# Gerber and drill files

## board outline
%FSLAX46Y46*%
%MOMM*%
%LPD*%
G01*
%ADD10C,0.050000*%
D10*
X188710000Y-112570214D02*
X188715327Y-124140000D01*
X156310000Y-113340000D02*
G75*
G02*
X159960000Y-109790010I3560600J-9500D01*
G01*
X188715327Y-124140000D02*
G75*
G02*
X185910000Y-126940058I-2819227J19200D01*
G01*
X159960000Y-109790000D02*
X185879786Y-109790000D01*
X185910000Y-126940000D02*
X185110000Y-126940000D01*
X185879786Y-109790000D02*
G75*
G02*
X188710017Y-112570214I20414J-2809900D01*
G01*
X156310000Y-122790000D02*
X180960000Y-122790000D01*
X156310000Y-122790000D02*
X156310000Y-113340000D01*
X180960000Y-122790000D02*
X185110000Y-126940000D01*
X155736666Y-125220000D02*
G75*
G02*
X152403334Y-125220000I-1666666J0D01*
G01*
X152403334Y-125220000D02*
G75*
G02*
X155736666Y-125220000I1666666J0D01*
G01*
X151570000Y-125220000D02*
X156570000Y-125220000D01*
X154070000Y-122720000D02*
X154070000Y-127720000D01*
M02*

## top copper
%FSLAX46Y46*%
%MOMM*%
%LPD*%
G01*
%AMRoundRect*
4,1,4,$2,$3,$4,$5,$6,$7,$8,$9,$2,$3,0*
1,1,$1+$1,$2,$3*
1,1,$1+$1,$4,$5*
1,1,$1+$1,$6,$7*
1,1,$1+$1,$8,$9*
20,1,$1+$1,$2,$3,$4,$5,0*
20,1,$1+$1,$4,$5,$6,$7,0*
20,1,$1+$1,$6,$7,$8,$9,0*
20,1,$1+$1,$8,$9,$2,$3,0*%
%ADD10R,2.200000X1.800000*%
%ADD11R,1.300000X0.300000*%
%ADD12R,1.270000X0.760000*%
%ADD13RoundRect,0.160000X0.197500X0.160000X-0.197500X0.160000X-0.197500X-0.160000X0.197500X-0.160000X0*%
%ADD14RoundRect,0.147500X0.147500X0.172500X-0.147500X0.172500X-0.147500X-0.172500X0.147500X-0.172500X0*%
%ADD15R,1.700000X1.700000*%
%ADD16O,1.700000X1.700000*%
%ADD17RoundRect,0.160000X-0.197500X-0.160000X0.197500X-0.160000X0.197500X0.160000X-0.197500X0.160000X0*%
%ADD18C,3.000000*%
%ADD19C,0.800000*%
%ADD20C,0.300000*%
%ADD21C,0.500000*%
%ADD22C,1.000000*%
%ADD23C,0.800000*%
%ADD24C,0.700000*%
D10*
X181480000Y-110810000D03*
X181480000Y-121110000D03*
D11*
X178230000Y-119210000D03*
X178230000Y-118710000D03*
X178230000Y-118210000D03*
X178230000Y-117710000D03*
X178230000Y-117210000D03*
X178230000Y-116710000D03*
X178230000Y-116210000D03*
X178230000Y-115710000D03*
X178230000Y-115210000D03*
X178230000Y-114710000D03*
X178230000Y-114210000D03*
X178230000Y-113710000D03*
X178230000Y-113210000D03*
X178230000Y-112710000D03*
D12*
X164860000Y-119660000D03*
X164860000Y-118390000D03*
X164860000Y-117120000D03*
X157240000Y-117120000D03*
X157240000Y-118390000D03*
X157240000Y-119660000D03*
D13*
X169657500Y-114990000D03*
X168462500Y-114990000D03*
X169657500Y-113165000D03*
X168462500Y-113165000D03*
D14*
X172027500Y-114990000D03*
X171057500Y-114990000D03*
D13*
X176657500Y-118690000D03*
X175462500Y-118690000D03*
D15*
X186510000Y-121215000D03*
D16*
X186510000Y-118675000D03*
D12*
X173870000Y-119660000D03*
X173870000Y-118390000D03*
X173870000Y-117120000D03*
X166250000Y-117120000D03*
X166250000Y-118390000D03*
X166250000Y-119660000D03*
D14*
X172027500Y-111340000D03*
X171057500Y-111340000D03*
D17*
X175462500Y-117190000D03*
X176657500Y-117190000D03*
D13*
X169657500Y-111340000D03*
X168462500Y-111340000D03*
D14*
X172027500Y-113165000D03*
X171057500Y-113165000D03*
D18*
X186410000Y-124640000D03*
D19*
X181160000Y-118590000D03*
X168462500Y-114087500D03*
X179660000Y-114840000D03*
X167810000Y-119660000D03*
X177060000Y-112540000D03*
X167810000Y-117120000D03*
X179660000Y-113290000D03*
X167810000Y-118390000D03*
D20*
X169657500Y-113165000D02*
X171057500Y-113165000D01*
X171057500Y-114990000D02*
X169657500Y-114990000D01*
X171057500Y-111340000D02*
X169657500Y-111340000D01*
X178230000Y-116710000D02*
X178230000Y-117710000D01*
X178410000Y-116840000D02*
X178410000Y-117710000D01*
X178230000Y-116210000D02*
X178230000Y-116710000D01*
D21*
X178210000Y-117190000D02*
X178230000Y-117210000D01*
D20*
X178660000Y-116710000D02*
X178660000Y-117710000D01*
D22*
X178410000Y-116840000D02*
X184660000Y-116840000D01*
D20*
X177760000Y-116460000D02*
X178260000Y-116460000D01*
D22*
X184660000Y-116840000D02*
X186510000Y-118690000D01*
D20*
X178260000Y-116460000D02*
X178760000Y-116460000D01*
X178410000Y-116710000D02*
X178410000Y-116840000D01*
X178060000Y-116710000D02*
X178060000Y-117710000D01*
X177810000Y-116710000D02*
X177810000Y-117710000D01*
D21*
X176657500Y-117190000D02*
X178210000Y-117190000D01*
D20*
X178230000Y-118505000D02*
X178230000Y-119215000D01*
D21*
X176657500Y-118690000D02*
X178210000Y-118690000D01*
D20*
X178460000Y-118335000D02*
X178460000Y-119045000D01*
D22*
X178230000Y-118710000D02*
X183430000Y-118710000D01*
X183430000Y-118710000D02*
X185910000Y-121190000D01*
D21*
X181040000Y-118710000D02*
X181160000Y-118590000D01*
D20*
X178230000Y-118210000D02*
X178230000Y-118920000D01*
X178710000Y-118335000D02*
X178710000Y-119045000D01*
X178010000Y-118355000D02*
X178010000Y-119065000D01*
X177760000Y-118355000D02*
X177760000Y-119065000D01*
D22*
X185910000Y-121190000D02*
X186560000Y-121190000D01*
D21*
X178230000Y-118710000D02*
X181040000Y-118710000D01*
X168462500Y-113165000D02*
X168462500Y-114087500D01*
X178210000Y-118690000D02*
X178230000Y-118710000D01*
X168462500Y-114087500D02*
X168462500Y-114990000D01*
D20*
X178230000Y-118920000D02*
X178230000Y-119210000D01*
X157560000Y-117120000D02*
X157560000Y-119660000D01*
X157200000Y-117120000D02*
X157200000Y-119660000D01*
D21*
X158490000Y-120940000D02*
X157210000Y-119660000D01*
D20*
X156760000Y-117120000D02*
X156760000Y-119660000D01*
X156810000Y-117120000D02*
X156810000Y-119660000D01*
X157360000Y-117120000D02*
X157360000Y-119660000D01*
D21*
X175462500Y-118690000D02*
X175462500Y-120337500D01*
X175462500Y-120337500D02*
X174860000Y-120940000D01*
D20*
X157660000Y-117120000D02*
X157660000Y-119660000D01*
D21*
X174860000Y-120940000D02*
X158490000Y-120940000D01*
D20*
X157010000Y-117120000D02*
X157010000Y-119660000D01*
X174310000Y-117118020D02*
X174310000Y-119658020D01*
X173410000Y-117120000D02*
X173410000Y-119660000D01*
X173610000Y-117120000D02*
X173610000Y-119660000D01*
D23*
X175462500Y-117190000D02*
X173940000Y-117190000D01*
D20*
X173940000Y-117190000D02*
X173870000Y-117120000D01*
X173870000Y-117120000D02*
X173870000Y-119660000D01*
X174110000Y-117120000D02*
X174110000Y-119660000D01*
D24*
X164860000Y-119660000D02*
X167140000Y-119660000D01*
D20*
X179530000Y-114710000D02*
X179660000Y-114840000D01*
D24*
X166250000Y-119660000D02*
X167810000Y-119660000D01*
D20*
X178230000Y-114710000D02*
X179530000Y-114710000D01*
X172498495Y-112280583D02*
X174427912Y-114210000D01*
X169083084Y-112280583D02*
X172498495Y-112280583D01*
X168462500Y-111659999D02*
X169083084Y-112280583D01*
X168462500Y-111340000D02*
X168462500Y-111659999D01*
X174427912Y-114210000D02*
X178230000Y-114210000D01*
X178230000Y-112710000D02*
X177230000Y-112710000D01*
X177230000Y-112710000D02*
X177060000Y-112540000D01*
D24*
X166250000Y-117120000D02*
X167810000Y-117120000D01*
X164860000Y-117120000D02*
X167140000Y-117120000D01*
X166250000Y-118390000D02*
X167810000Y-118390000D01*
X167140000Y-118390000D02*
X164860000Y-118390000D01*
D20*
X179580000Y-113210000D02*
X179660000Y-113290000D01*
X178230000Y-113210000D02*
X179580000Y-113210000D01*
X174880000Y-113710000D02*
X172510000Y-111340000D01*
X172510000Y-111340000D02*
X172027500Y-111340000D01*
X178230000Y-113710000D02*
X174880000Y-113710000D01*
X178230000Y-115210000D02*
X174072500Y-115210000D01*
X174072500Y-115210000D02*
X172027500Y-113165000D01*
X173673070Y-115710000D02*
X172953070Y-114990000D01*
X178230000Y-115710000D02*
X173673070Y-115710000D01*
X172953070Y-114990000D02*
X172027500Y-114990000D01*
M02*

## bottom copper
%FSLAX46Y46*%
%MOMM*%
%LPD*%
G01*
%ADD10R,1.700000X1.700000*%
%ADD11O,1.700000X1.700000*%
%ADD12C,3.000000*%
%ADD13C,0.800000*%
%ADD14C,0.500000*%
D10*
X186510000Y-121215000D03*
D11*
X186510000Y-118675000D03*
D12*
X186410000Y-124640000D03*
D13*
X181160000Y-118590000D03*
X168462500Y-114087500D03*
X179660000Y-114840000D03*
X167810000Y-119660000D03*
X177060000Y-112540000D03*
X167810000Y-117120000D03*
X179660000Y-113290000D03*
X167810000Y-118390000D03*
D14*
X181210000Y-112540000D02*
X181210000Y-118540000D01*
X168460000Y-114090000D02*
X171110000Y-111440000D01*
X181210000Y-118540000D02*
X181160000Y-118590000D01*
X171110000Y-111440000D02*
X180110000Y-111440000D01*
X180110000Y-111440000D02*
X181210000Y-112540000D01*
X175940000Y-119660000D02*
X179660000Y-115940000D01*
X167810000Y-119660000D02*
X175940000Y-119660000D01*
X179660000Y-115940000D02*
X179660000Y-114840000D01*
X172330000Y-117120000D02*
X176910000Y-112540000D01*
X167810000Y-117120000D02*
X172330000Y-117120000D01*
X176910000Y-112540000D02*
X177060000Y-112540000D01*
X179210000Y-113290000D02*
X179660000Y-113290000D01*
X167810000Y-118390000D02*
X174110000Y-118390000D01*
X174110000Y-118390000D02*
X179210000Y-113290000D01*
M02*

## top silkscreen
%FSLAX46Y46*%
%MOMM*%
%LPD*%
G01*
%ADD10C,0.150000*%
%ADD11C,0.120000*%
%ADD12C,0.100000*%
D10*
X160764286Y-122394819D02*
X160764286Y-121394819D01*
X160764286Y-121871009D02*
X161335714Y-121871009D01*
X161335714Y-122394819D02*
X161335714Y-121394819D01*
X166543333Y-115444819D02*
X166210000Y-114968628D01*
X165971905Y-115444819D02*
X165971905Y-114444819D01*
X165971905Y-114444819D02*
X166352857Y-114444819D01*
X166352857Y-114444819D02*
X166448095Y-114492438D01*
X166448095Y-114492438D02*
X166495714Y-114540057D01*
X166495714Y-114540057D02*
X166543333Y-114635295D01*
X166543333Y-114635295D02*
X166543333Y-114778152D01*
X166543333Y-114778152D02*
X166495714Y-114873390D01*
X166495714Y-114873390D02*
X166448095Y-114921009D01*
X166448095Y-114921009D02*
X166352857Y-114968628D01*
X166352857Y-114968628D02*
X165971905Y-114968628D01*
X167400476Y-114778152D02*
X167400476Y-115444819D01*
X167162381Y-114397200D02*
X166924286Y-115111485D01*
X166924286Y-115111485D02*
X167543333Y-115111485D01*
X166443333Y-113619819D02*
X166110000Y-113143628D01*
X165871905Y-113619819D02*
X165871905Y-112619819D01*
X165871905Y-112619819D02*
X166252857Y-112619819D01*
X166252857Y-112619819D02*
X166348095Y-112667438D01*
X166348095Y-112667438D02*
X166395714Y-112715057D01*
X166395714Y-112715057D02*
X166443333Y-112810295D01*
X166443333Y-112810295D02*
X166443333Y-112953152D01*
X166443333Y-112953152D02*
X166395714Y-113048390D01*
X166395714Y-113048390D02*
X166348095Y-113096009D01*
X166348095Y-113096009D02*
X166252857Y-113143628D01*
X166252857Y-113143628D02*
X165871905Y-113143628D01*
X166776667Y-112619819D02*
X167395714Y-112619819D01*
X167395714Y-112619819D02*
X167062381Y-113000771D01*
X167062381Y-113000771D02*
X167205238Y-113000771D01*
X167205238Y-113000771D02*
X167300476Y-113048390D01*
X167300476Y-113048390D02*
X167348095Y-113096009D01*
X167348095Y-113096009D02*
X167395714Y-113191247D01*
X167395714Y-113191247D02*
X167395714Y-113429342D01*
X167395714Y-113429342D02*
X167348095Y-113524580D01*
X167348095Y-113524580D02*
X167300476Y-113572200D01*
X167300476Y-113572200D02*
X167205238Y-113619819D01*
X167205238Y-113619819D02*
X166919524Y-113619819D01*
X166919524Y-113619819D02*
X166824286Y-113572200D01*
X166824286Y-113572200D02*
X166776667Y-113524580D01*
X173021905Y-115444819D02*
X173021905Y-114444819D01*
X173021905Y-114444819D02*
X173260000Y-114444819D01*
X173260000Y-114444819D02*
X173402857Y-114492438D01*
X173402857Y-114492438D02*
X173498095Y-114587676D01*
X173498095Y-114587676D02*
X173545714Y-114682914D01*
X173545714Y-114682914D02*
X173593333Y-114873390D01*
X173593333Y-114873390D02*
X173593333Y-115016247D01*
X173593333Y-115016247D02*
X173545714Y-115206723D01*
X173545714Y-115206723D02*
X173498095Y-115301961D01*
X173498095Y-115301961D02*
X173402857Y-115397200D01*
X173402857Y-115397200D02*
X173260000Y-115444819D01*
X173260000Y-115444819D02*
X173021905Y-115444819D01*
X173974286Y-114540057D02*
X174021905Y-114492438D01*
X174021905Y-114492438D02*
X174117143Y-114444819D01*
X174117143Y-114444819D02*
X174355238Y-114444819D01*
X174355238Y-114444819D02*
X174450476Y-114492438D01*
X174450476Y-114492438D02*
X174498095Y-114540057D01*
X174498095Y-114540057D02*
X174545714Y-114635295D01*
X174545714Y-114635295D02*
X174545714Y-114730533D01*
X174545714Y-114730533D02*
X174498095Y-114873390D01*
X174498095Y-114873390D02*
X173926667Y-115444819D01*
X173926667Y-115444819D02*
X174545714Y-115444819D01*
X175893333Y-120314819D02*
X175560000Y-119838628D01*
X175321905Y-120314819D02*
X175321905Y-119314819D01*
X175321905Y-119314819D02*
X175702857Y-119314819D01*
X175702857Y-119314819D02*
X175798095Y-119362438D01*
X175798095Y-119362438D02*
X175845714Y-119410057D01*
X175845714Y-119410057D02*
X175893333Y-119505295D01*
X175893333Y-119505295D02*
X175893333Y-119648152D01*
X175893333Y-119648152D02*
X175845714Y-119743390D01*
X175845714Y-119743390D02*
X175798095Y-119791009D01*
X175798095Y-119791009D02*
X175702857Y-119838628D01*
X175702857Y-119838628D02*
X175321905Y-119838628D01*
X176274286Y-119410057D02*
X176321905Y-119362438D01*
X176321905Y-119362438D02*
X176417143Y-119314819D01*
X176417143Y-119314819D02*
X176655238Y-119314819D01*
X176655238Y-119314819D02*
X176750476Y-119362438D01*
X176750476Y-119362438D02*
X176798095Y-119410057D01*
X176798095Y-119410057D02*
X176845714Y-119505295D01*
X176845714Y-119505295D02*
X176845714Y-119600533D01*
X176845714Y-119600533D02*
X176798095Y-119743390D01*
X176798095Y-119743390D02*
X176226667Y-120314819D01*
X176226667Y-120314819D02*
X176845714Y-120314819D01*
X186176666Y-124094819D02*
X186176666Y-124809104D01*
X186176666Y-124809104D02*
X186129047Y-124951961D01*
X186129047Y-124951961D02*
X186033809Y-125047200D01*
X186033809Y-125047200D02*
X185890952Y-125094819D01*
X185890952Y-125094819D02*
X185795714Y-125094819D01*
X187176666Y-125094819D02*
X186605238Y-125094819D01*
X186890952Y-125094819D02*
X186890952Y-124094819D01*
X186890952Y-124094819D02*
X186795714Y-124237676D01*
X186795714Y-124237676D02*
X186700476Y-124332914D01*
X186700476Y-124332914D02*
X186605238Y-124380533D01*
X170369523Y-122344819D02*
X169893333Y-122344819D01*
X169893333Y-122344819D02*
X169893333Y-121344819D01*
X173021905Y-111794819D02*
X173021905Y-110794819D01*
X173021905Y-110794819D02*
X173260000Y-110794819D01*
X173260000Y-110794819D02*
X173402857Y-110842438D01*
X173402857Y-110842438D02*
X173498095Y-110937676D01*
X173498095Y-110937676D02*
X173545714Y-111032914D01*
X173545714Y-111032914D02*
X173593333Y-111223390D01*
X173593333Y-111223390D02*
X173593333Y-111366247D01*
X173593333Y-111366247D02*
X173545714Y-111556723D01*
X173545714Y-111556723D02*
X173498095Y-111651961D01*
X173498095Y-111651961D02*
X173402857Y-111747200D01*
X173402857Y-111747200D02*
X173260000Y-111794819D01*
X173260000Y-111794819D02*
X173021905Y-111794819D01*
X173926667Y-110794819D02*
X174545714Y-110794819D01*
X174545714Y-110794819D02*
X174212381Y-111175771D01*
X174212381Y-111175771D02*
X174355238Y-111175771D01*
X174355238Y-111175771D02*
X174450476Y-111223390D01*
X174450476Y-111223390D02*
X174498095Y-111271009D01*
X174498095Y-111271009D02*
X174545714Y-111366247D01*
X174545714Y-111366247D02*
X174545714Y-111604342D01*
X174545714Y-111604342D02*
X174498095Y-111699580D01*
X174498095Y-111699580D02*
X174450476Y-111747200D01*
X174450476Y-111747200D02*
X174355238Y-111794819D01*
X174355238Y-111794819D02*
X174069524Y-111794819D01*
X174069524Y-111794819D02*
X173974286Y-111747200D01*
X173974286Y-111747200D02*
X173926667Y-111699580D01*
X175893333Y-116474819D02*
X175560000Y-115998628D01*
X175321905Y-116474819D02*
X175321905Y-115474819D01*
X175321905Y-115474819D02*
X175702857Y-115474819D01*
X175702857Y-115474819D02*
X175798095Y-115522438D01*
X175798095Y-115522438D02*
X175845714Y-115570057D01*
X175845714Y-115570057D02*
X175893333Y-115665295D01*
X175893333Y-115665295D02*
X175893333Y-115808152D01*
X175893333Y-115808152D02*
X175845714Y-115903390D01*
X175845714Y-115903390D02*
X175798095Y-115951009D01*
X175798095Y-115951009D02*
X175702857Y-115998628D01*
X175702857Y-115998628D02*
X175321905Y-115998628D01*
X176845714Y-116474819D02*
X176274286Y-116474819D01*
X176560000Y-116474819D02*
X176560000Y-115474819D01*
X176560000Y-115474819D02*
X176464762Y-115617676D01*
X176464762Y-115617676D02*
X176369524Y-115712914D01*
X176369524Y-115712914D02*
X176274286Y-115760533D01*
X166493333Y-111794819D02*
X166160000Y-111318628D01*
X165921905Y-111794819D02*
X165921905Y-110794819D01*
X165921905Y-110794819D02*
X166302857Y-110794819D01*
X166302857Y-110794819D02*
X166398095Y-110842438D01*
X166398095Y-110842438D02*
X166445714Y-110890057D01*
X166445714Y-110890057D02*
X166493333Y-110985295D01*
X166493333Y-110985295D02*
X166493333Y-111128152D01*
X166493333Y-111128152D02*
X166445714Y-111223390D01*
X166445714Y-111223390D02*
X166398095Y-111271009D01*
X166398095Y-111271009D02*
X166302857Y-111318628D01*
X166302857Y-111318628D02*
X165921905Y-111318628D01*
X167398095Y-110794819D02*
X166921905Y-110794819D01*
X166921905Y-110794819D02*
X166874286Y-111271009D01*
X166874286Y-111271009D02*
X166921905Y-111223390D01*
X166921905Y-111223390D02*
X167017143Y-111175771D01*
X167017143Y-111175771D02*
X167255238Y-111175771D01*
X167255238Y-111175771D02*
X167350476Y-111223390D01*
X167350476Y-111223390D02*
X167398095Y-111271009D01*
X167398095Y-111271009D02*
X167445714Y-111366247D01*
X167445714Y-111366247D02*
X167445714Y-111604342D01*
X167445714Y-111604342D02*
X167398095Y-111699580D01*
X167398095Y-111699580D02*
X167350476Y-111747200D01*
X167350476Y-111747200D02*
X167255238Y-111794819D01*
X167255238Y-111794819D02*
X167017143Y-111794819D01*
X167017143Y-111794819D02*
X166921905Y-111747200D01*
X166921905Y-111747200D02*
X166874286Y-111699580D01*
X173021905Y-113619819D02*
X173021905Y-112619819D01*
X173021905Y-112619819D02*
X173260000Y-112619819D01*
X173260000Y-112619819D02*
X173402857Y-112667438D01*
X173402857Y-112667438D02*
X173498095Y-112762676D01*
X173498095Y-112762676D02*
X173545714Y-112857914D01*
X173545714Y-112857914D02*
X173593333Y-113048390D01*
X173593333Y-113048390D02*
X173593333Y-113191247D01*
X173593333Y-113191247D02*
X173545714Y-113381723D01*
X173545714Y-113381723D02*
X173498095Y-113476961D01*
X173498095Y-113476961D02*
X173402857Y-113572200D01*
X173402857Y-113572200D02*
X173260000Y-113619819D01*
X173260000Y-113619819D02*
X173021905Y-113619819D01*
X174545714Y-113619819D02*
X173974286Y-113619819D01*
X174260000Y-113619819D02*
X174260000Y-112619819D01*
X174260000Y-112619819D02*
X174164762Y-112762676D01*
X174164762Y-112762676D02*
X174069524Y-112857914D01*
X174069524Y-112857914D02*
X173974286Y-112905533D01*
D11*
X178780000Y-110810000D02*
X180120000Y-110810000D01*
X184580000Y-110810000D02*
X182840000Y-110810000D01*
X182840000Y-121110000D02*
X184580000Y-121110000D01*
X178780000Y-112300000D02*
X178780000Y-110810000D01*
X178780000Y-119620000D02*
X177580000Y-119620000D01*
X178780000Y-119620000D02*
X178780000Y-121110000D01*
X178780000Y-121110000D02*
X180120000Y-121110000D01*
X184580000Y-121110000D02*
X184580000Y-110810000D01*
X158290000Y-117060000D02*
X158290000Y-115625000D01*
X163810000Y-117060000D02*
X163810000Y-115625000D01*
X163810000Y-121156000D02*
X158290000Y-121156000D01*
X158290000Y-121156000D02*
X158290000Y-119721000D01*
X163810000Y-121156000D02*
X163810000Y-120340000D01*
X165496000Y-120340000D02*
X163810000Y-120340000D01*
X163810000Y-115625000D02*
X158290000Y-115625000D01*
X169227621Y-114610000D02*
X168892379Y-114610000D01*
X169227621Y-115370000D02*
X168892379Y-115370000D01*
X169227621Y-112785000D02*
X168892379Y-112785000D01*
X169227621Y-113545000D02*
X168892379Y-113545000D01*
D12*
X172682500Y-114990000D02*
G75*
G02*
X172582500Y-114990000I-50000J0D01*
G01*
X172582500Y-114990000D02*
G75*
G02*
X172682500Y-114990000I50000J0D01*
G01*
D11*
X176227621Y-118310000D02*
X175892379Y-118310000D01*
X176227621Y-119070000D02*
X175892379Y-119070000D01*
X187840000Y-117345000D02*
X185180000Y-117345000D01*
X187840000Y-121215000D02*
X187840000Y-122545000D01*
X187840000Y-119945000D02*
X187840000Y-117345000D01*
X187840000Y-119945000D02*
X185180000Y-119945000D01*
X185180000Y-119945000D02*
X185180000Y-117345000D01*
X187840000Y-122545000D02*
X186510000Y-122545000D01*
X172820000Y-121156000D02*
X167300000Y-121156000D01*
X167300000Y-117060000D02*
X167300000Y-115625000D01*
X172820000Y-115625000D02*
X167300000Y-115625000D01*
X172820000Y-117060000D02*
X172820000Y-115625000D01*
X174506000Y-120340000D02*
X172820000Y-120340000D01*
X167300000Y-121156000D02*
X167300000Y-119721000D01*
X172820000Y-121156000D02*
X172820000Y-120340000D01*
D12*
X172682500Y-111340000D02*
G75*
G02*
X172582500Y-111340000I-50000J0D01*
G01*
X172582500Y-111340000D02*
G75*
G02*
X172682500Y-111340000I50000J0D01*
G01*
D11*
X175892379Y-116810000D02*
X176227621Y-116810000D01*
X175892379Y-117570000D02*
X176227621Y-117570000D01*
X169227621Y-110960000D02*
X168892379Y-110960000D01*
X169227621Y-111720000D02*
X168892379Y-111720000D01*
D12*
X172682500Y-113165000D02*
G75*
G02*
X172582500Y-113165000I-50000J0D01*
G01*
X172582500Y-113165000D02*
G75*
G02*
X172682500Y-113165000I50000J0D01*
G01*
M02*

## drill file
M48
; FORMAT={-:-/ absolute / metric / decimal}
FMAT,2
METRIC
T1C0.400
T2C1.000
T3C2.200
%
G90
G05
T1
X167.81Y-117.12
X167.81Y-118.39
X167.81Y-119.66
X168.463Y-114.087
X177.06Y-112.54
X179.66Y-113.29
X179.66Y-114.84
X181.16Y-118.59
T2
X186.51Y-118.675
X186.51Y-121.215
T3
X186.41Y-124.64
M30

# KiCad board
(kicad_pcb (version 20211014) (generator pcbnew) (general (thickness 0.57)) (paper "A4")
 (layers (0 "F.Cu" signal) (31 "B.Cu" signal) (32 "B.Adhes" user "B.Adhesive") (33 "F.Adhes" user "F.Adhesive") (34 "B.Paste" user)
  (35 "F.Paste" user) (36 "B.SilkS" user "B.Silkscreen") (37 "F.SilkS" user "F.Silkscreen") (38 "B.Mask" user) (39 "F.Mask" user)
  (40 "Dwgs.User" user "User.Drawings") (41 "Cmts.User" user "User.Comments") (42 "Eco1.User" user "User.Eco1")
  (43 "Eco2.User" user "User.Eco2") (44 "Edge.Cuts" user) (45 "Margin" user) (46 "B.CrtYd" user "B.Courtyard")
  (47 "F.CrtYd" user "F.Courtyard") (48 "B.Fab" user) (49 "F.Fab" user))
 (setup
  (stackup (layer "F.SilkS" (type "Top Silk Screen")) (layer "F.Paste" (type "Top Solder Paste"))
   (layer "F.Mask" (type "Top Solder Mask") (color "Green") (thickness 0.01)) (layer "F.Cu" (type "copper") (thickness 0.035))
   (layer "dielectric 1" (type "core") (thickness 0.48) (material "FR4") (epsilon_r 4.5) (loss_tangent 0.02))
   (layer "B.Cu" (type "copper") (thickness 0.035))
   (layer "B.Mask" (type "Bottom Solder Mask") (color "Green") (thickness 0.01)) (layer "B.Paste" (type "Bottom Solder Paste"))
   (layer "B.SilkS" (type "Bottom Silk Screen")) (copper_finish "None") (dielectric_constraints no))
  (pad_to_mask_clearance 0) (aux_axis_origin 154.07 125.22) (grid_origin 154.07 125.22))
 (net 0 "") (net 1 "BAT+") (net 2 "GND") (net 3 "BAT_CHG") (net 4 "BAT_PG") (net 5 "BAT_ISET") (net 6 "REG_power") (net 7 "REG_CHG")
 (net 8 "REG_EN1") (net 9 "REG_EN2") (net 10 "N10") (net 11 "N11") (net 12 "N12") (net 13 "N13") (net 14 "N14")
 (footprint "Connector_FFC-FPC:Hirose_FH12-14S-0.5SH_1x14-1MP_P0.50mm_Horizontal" (layer "F.Cu") (at 180.08 115.96 90)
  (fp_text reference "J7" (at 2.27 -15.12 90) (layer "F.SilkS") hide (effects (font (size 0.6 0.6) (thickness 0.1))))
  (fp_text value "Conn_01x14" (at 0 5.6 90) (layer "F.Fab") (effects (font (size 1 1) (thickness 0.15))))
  (fp_line (start 5.15 -1.3) (end 5.15 0.04) (layer "F.SilkS") (width 0.12))
  (fp_line (start 5.15 4.5) (end 5.15 2.76) (layer "F.SilkS") (width 0.12))
  (fp_line (start -5.15 2.76) (end -5.15 4.5) (layer "F.SilkS") (width 0.12))
  (fp_line (start 3.66 -1.3) (end 5.15 -1.3) (layer "F.SilkS") (width 0.12))
  (fp_line (start -3.66 -1.3) (end -3.66 -2.5) (layer "F.SilkS") (width 0.12))
  (fp_line (start -3.66 -1.3) (end -5.15 -1.3) (layer "F.SilkS") (width 0.12))
  (fp_line (start -5.15 -1.3) (end -5.15 0.04) (layer "F.SilkS") (width 0.12))
  (fp_line (start -5.15 4.5) (end 5.15 4.5) (layer "F.SilkS") (width 0.12))
  (pad "" smd rect (at 5.15 1.4 90) (size 1.8 2.2) (layers "F.Cu" "F.Paste" "F.Mask"))
  (pad "" smd rect (at -5.15 1.4 90) (size 1.8 2.2) (layers "F.Cu" "F.Paste" "F.Mask"))
  (pad "1" smd rect (at -3.25 -1.85 90) (size 0.3 1.3) (layers "F.Cu" "F.Paste" "F.Mask") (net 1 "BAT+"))
  (pad "2" smd rect (at -2.75 -1.85 90) (size 0.3 1.3) (layers "F.Cu" "F.Paste" "F.Mask") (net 1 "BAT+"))
  (pad "3" smd rect (at -2.25 -1.85 90) (size 0.3 1.3) (layers "F.Cu" "F.Paste" "F.Mask") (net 1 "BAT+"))
  (pad "4" smd rect (at -1.75 -1.85 90) (size 0.3 1.3) (layers "F.Cu" "F.Paste" "F.Mask") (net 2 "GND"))
  (pad "5" smd rect (at -1.25 -1.85 90) (size 0.3 1.3) (layers "F.Cu" "F.Paste" "F.Mask") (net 2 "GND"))
  (pad "6" smd rect (at -0.75 -1.85 90) (size 0.3 1.3) (layers "F.Cu" "F.Paste" "F.Mask") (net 2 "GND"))
  (pad "7" smd rect (at -0.25 -1.85 90) (size 0.3 1.3) (layers "F.Cu" "F.Paste" "F.Mask") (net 2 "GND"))
  (pad "8" smd rect (at 0.25 -1.85 90) (size 0.3 1.3) (layers "F.Cu" "F.Paste" "F.Mask") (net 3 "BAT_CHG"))
  (pad "9" smd rect (at 0.75 -1.85 90) (size 0.3 1.3) (layers "F.Cu" "F.Paste" "F.Mask") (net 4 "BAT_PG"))
  (pad "10" smd rect (at 1.25 -1.85 90) (size 0.3 1.3) (layers "F.Cu" "F.Paste" "F.Mask") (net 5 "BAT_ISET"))
  (pad "11" smd rect (at 1.75 -1.85 90) (size 0.3 1.3) (layers "F.Cu" "F.Paste" "F.Mask") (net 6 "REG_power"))
  (pad "12" smd rect (at 2.25 -1.85 90) (size 0.3 1.3) (layers "F.Cu" "F.Paste" "F.Mask") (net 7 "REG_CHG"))
  (pad "13" smd rect (at 2.75 -1.85 90) (size 0.3 1.3) (layers "F.Cu" "F.Paste" "F.Mask") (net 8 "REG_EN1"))
  (pad "14" smd rect (at 3.25 -1.85 90) (size 0.3 1.3) (layers "F.Cu" "F.Paste" "F.Mask") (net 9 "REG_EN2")))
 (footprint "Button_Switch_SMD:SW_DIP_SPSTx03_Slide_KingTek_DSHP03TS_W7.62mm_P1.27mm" (layer "F.Cu") (at 161.05 118.39 180)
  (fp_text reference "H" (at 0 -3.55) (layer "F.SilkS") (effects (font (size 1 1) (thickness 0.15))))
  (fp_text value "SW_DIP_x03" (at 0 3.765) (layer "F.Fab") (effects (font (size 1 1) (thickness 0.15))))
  (fp_line (start 2.76 1.33) (end 2.76 2.765) (layer "F.SilkS") (width 0.12))
  (fp_line (start -2.76 1.33) (end -2.76 2.765) (layer "F.SilkS") (width 0.12))
  (fp_line (start -2.76 -2.766) (end 2.76 -2.766) (layer "F.SilkS") (width 0.12))
  (fp_line (start 2.76 -2.766) (end 2.76 -1.331) (layer "F.SilkS") (width 0.12))
  (fp_line (start -2.76 -2.766) (end -2.76 -1.95) (layer "F.SilkS") (width 0.12))
  (fp_line (start -4.446 -1.95) (end -2.76 -1.95) (layer "F.SilkS") (width 0.12))
  (fp_line (start -2.76 2.765) (end 2.76 2.765) (layer "F.SilkS") (width 0.12))
  (pad "1" smd rect locked (at -3.81 -1.27 180) (size 1.27 0.76) (layers "F.Cu" "F.Paste" "F.Mask") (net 5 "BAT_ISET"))
  (pad "2" smd rect locked (at -3.81 0 180) (size 1.27 0.76) (layers "F.Cu" "F.Paste" "F.Mask") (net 8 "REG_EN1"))
  (pad "3" smd rect locked (at -3.81 1.27 180) (size 1.27 0.76) (layers "F.Cu" "F.Paste" "F.Mask") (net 9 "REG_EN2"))
  (pad "4" smd rect locked (at 3.81 1.27 180) (size 1.27 0.76) (layers "F.Cu" "F.Paste" "F.Mask") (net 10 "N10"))
  (pad "5" smd rect locked (at 3.81 0 180) (size 1.27 0.76) (layers "F.Cu" "F.Paste" "F.Mask") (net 10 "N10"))
  (pad "6" smd rect locked (at 3.81 -1.27 180) (size 1.27 0.76) (layers "F.Cu" "F.Paste" "F.Mask") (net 10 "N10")))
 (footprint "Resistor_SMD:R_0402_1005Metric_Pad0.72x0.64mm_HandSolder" (layer "F.Cu") (at 169.06 114.99 180)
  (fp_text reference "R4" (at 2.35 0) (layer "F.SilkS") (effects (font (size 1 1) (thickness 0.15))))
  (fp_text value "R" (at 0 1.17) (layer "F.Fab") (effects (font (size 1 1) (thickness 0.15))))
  (fp_line (start -0.167621 0.38) (end 0.167621 0.38) (layer "F.SilkS") (width 0.12))
  (fp_line (start -0.167621 -0.38) (end 0.167621 -0.38) (layer "F.SilkS") (width 0.12))
  (pad "1" smd roundrect locked (at -0.5975 0 180) (size 0.715 0.64) (layers "F.Cu" "F.Paste" "F.Mask") (roundrect_rratio 0.25)
   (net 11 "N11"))
  (pad "2" smd roundrect locked (at 0.5975 0 180) (size 0.715 0.64) (layers "F.Cu" "F.Paste" "F.Mask") (roundrect_rratio 0.25)
   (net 1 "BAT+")))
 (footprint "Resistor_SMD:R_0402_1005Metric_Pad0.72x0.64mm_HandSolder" (layer "F.Cu") (at 169.06 113.165 180)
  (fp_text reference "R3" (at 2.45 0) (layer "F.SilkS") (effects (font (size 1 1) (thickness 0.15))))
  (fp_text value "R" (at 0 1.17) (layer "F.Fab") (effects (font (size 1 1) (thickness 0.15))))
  (fp_line (start -0.167621 0.38) (end 0.167621 0.38) (layer "F.SilkS") (width 0.12))
  (fp_line (start -0.167621 -0.38) (end 0.167621 -0.38) (layer "F.SilkS") (width 0.12))
  (pad "1" smd roundrect locked (at -0.5975 0 180) (size 0.715 0.64) (layers "F.Cu" "F.Paste" "F.Mask") (roundrect_rratio 0.25)
   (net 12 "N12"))
  (pad "2" smd roundrect locked (at 0.5975 0 180) (size 0.715 0.64) (layers "F.Cu" "F.Paste" "F.Mask") (roundrect_rratio 0.25)
   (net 1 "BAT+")))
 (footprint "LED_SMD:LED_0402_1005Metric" (layer "F.Cu") (at 171.5425 114.99 180)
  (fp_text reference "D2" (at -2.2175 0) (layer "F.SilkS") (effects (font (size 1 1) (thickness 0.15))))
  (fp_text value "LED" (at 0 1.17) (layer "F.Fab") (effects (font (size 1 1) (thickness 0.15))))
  (fp_circle (center -1.09 0) (end -1.04 0) (layer "F.SilkS") (width 0.1) (fill none))
  (pad "1" smd roundrect locked (at -0.485 0 180) (size 0.59 0.64) (layers "F.Cu" "F.Paste" "F.Mask") (roundrect_rratio 0.25)
   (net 3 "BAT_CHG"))
  (pad "2" smd roundrect locked (at 0.485 0 180) (size 0.59 0.64) (layers "F.Cu" "F.Paste" "F.Mask") (roundrect_rratio 0.25) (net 11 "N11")))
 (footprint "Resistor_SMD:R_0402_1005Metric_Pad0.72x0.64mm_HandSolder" (layer "F.Cu") (at 176.06 118.69 180)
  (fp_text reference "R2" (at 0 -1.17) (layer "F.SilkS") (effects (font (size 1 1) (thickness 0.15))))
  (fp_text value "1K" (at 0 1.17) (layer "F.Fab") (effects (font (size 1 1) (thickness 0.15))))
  (fp_line (start -0.167621 0.38) (end 0.167621 0.38) (layer "F.SilkS") (width 0.12))
  (fp_line (start -0.167621 -0.38) (end 0.167621 -0.38) (layer "F.SilkS") (width 0.12))
  (pad "1" smd roundrect locked (at -0.5975 0 180) (size 0.715 0.64) (layers "F.Cu" "F.Paste" "F.Mask") (roundrect_rratio 0.25)
   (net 1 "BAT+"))
  (pad "2" smd roundrect locked (at 0.5975 0 180) (size 0.715 0.64) (layers "F.Cu" "F.Paste" "F.Mask") (roundrect_rratio 0.25)
   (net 10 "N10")))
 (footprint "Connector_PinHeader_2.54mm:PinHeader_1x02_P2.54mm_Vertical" (layer "F.Cu") (at 186.51 121.215 180)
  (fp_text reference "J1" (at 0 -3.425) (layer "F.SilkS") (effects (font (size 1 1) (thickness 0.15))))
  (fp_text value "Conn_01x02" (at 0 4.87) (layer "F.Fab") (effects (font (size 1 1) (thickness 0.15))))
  (fp_line (start -1.33 3.87) (end 1.33 3.87) (layer "F.SilkS") (width 0.12))
  (fp_line (start -1.33 0) (end -1.33 -1.33) (layer "F.SilkS") (width 0.12))
  (fp_line (start -1.33 1.27) (end -1.33 3.87) (layer "F.SilkS") (width 0.12))
  (fp_line (start -1.33 1.27) (end 1.33 1.27) (layer "F.SilkS") (width 0.12))
  (fp_line (start 1.33 1.27) (end 1.33 3.87) (layer "F.SilkS") (width 0.12))
  (fp_line (start -1.33 -1.33) (end 0 -1.33) (layer "F.SilkS") (width 0.12))
  (pad "1" thru_hole rect locked (at 0 0 180) (size 1.7 1.7) (drill 1) (layers *.Cu *.Mask) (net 1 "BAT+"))
  (pad "2" thru_hole oval locked (at 0 2.54 180) (size 1.7 1.7) (drill 1) (layers *.Cu *.Mask) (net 2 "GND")))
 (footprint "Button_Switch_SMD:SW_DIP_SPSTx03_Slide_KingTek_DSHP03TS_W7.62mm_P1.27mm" (layer "F.Cu") (at 170.06 118.39 180)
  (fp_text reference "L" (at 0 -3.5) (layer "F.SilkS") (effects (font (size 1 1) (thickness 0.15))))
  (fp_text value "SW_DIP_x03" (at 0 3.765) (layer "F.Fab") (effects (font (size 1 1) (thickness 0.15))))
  (fp_line (start -2.76 -2.766) (end 2.76 -2.766) (layer "F.SilkS") (width 0.12))
  (fp_line (start 2.76 1.33) (end 2.76 2.765) (layer "F.SilkS") (width 0.12))
  (fp_line (start -2.76 2.765) (end 2.76 2.765) (layer "F.SilkS") (width 0.12))
  (fp_line (start -2.76 1.33) (end -2.76 2.765) (layer "F.SilkS") (width 0.12))
  (fp_line (start -4.446 -1.95) (end -2.76 -1.95) (layer "F.SilkS") (width 0.12))
  (fp_line (start 2.76 -2.766) (end 2.76 -1.331) (layer "F.SilkS") (width 0.12))
  (fp_line (start -2.76 -2.766) (end -2.76 -1.95) (layer "F.SilkS") (width 0.12))
  (pad "1" smd rect locked (at -3.81 -1.27 180) (size 1.27 0.76) (layers "F.Cu" "F.Paste" "F.Mask") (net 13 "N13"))
  (pad "2" smd rect locked (at -3.81 0 180) (size 1.27 0.76) (layers "F.Cu" "F.Paste" "F.Mask") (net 13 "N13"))
  (pad "3" smd rect locked (at -3.81 1.27 180) (size 1.27 0.76) (layers "F.Cu" "F.Paste" "F.Mask") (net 13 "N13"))
  (pad "4" smd rect locked (at 3.81 1.27 180) (size 1.27 0.76) (layers "F.Cu" "F.Paste" "F.Mask") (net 9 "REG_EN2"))
  (pad "5" smd rect locked (at 3.81 0 180) (size 1.27 0.76) (layers "F.Cu" "F.Paste" "F.Mask") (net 8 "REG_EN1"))
  (pad "6" smd rect locked (at 3.81 -1.27 180) (size 1.27 0.76) (layers "F.Cu" "F.Paste" "F.Mask") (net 5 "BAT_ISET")))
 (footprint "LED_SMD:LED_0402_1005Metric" (layer "F.Cu") (at 171.5425 111.34 180)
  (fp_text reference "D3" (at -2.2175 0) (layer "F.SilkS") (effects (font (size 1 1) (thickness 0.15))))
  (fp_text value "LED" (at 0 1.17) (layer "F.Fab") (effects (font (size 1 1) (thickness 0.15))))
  (fp_circle (center -1.09 0) (end -1.04 0) (layer "F.SilkS") (width 0.1) (fill none))
  (pad "1" smd roundrect locked (at -0.485 0 180) (size 0.59 0.64) (layers "F.Cu" "F.Paste" "F.Mask") (roundrect_rratio 0.25)
   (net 7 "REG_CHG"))
  (pad "2" smd roundrect locked (at 0.485 0 180) (size 0.59 0.64) (layers "F.Cu" "F.Paste" "F.Mask") (roundrect_rratio 0.25) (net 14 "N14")))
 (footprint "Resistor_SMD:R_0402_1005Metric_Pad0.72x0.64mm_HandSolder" (layer "F.Cu") (at 176.06 117.19)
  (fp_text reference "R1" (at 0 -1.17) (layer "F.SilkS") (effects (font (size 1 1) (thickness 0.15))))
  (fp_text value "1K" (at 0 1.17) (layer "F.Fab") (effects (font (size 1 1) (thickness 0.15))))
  (fp_line (start -0.167621 -0.38) (end 0.167621 -0.38) (layer "F.SilkS") (width 0.12))
  (fp_line (start -0.167621 0.38) (end 0.167621 0.38) (layer "F.SilkS") (width 0.12))
  (pad "1" smd roundrect locked (at -0.5975 0) (size 0.715 0.64) (layers "F.Cu" "F.Paste" "F.Mask") (roundrect_rratio 0.25) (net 13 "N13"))
  (pad "2" smd roundrect locked (at 0.5975 0) (size 0.715 0.64) (layers "F.Cu" "F.Paste" "F.Mask") (roundrect_rratio 0.25) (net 2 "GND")))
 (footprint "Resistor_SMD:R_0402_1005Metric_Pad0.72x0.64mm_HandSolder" (layer "F.Cu") (at 169.06 111.34 180)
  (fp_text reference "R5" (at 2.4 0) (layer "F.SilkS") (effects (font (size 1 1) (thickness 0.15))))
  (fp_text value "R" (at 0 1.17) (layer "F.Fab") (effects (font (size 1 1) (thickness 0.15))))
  (fp_line (start -0.167621 0.38) (end 0.167621 0.38) (layer "F.SilkS") (width 0.12))
  (fp_line (start -0.167621 -0.38) (end 0.167621 -0.38) (layer "F.SilkS") (width 0.12))
  (pad "1" smd roundrect locked (at -0.5975 0 180) (size 0.715 0.64) (layers "F.Cu" "F.Paste" "F.Mask") (roundrect_rratio 0.25)
   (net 14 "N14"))
  (pad "2" smd roundrect locked (at 0.5975 0 180) (size 0.715 0.64) (layers "F.Cu" "F.Paste" "F.Mask") (roundrect_rratio 0.25)
   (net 6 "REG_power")))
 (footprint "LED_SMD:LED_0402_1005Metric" (layer "F.Cu") (at 171.5425 113.165 180)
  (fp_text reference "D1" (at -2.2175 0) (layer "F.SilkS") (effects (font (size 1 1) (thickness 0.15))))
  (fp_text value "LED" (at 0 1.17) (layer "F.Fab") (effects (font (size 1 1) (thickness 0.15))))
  (fp_circle (center -1.09 0) (end -1.04 0) (layer "F.SilkS") (width 0.1) (fill none))
  (pad "1" smd roundrect locked (at -0.485 0 180) (size 0.59 0.64) (layers "F.Cu" "F.Paste" "F.Mask") (roundrect_rratio 0.25)
   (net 4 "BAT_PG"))
  (pad "2" smd roundrect locked (at 0.485 0 180) (size 0.59 0.64) (layers "F.Cu" "F.Paste" "F.Mask") (roundrect_rratio 0.25) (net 12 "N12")))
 (gr_line (start 188.71 112.570214) (end 188.715327 124.14) (layer "Edge.Cuts") (width 0.05))
 (gr_arc (start 156.31 113.34) (mid 157.38808 110.79704) (end 159.96 109.79) (layer "Edge.Cuts") (width 0.05))
 (gr_arc (start 188.715327 124.14) (mid 187.887752 126.116183) (end 185.91 126.94) (layer "Edge.Cuts") (width 0.05))
 (gr_line (start 159.96 109.79) (end 185.879786 109.79) (layer "Edge.Cuts") (width 0.05))
 (gr_line (start 185.91 126.94) (end 185.11 126.94) (layer "Edge.Cuts") (width 0.05))
 (gr_arc (start 185.879786 109.79) (mid 187.869341 110.595328) (end 188.71 112.570214) (layer "Edge.Cuts") (width 0.05))
 (gr_line (start 156.31 122.79) (end 180.96 122.79) (layer "Edge.Cuts") (width 0.05))
 (gr_line (start 156.31 122.79) (end 156.31 113.34) (layer "Edge.Cuts") (width 0.05))
 (gr_line (start 180.96 122.79) (end 185.11 126.94) (layer "Edge.Cuts") (width 0.05))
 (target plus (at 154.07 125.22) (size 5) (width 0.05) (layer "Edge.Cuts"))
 (via (at 186.41 124.64) (size 3) (drill 2.2) (layers "F.Cu" "B.Cu") (free) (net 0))
 (segment (start 169.6575 113.165) (end 171.0575 113.165) (width 0.3) (layer "F.Cu") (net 12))
 (segment (start 171.0575 114.99) (end 169.6575 114.99) (width 0.3) (layer "F.Cu") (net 11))
 (segment (start 171.0575 111.34) (end 169.6575 111.34) (width 0.3) (layer "F.Cu") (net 14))
 (segment (start 178.23 116.71) (end 178.23 117.71) (width 0.3) (layer "F.Cu") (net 2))
 (segment (start 178.41 116.84) (end 178.41 117.71) (width 0.3) (layer "F.Cu") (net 2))
 (segment (start 178.23 116.21) (end 178.23 116.71) (width 0.3) (layer "F.Cu") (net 2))
 (segment (start 178.21 117.19) (end 178.23 117.21) (width 0.5) (layer "F.Cu") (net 2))
 (segment (start 178.66 116.71) (end 178.66 117.71) (width 0.3) (layer "F.Cu") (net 2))
 (segment (start 178.41 116.84) (end 184.66 116.84) (width 1) (layer "F.Cu") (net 2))
 (segment (start 177.76 116.46) (end 178.26 116.46) (width 0.3) (layer "F.Cu") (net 2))
 (segment (start 184.66 116.84) (end 186.51 118.69) (width 1) (layer "F.Cu") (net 2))
 (segment (start 178.26 116.46) (end 178.76 116.46) (width 0.3) (layer "F.Cu") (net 2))
 (segment (start 178.41 116.71) (end 178.41 116.84) (width 0.3) (layer "F.Cu") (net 2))
 (segment (start 178.06 116.71) (end 178.06 117.71) (width 0.3) (layer "F.Cu") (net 2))
 (segment (start 177.81 116.71) (end 177.81 117.71) (width 0.3) (layer "F.Cu") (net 2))
 (segment (start 176.6575 117.19) (end 178.21 117.19) (width 0.5) (layer "F.Cu") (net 2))
 (segment (start 178.23 118.505) (end 178.23 119.215) (width 0.3) (layer "F.Cu") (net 1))
 (segment (start 176.6575 118.69) (end 178.21 118.69) (width 0.5) (layer "F.Cu") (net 1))
 (segment (start 178.46 118.335) (end 178.46 119.045) (width 0.3) (layer "F.Cu") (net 1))
 (segment (start 178.23 118.71) (end 183.43 118.71) (width 1) (layer "F.Cu") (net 1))
 (segment (start 183.43 118.71) (end 185.91 121.19) (width 1) (layer "F.Cu") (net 1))
 (segment (start 181.04 118.71) (end 181.16 118.59) (width 0.5) (layer "F.Cu") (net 1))
 (segment (start 178.23 118.21) (end 178.23 118.92) (width 0.3) (layer "F.Cu") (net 1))
 (segment (start 178.71 118.335) (end 178.71 119.045) (width 0.3) (layer "F.Cu") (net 1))
 (segment (start 178.01 118.355) (end 178.01 119.065) (width 0.3) (layer "F.Cu") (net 1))
 (segment (start 177.76 118.355) (end 177.76 119.065) (width 0.3) (layer "F.Cu") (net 1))
 (segment (start 185.91 121.19) (end 186.56 121.19) (width 1) (layer "F.Cu") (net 1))
 (segment (start 178.23 118.71) (end 181.04 118.71) (width 0.5) (layer "F.Cu") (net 1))
 (segment (start 168.4625 113.165) (end 168.4625 114.0875) (width 0.5) (layer "F.Cu") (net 1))
 (segment (start 178.21 118.69) (end 178.23 118.71) (width 0.5) (layer "F.Cu") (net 1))
 (segment (start 168.4625 114.0875) (end 168.4625 114.99) (width 0.5) (layer "F.Cu") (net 1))
 (segment (start 178.23 118.92) (end 178.23 119.21) (width 0.3) (layer "F.Cu") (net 1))
 (via (at 181.16 118.59) (size 0.8) (drill 0.4) (layers "F.Cu" "B.Cu") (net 1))
 (via (at 168.4625 114.0875) (size 0.8) (drill 0.4) (layers "F.Cu" "B.Cu") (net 1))
 (segment (start 181.21 112.54) (end 181.21 118.54) (width 0.5) (layer "B.Cu") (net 1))
 (segment (start 168.46 114.09) (end 171.11 111.44) (width 0.5) (layer "B.Cu") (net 1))
 (segment (start 181.21 118.54) (end 181.16 118.59) (width 0.5) (layer "B.Cu") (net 1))
 (segment (start 171.11 111.44) (end 180.11 111.44) (width 0.5) (layer "B.Cu") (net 1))
 (segment (start 180.11 111.44) (end 181.21 112.54) (width 0.5) (layer "B.Cu") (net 1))
 (segment (start 157.56 117.12) (end 157.56 119.66) (width 0.3) (layer "F.Cu") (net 10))
 (segment (start 157.2 117.12) (end 157.2 119.66) (width 0.3) (layer "F.Cu") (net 10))
 (segment (start 158.49 120.94) (end 157.21 119.66) (width 0.5) (layer "F.Cu") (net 10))
 (segment (start 156.76 117.12) (end 156.76 119.66) (width 0.3) (layer "F.Cu") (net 10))
 (segment (start 156.81 117.12) (end 156.81 119.66) (width 0.3) (layer "F.Cu") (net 10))
 (segment (start 157.36 117.12) (end 157.36 119.66) (width 0.3) (layer "F.Cu") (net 10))
 (segment (start 175.4625 118.69) (end 175.4625 120.3375) (width 0.5) (layer "F.Cu") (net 10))
 (segment (start 175.4625 120.3375) (end 174.86 120.94) (width 0.5) (layer "F.Cu") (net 10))
 (segment (start 157.66 117.12) (end 157.66 119.66) (width 0.3) (layer "F.Cu") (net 10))
 (segment (start 174.86 120.94) (end 158.49 120.94) (width 0.5) (layer "F.Cu") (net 10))
 (segment (start 157.01 117.12) (end 157.01 119.66) (width 0.3) (layer "F.Cu") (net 10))
 (segment (start 174.31 117.11802) (end 174.31 119.65802) (width 0.3) (layer "F.Cu") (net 13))
 (segment (start 173.41 117.12) (end 173.41 119.66) (width 0.3) (layer "F.Cu") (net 13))
 (segment (start 173.61 117.12) (end 173.61 119.66) (width 0.3) (layer "F.Cu") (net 13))
 (segment (start 175.4625 117.19) (end 173.94 117.19) (width 0.8) (layer "F.Cu") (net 13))
 (segment (start 173.94 117.19) (end 173.87 117.12) (width 0.3) (layer "F.Cu") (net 13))
 (segment (start 173.87 117.12) (end 173.87 119.66) (width 0.3) (layer "F.Cu") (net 13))
 (segment (start 174.11 117.12) (end 174.11 119.66) (width 0.3) (layer "F.Cu") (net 13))
 (segment (start 164.86 119.66) (end 167.14 119.66) (width 0.7) (layer "F.Cu") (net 5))
 (segment (start 179.53 114.71) (end 179.66 114.84) (width 0.3) (layer "F.Cu") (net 5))
 (segment (start 166.25 119.66) (end 167.81 119.66) (width 0.7) (layer "F.Cu") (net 5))
 (segment (start 178.23 114.71) (end 179.53 114.71) (width 0.3) (layer "F.Cu") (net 5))
 (via (at 179.66 114.84) (size 0.8) (drill 0.4) (layers "F.Cu" "B.Cu") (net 5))
 (via (at 167.81 119.66) (size 0.8) (drill 0.4) (layers "F.Cu" "B.Cu") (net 5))
 (segment (start 175.94 119.66) (end 179.66 115.94) (width 0.5) (layer "B.Cu") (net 5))
 (segment (start 167.81 119.66) (end 175.94 119.66) (width 0.5) (layer "B.Cu") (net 5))
 (segment (start 179.66 115.94) (end 179.66 114.84) (width 0.5) (layer "B.Cu") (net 5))
 (segment (start 172.498495 112.280583) (end 174.427912 114.21) (width 0.3) (layer "F.Cu") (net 6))
 (segment (start 169.083084 112.280583) (end 172.498495 112.280583) (width 0.3) (layer "F.Cu") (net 6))
 (segment (start 168.4625 111.659999) (end 169.083084 112.280583) (width 0.3) (layer "F.Cu") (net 6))
 (segment (start 168.4625 111.34) (end 168.4625 111.659999) (width 0.3) (layer "F.Cu") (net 6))
 (segment (start 174.427912 114.21) (end 178.23 114.21) (width 0.3) (layer "F.Cu") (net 6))
 (segment (start 178.23 112.71) (end 177.23 112.71) (width 0.3) (layer "F.Cu") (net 9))
 (segment (start 177.23 112.71) (end 177.06 112.54) (width 0.3) (layer "F.Cu") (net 9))
 (segment (start 166.25 117.12) (end 167.81 117.12) (width 0.7) (layer "F.Cu") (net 9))
 (segment (start 164.86 117.12) (end 167.14 117.12) (width 0.7) (layer "F.Cu") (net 9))
 (via (at 177.06 112.54) (size 0.8) (drill 0.4) (layers "F.Cu" "B.Cu") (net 9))
 (via (at 167.81 117.12) (size 0.8) (drill 0.4) (layers "F.Cu" "B.Cu") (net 9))
 (segment (start 172.33 117.12) (end 176.91 112.54) (width 0.5) (layer "B.Cu") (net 9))
 (segment (start 167.81 117.12) (end 172.33 117.12) (width 0.5) (layer "B.Cu") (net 9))
 (segment (start 176.91 112.54) (end 177.06 112.54) (width 0.5) (layer "B.Cu") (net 9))
 (segment (start 166.25 118.39) (end 167.81 118.39) (width 0.7) (layer "F.Cu") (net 8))
 (segment (start 167.14 118.39) (end 164.86 118.39) (width 0.7) (layer "F.Cu") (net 8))
 (segment (start 179.58 113.21) (end 179.66 113.29) (width 0.3) (layer "F.Cu") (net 8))
 (segment (start 178.23 113.21) (end 179.58 113.21) (width 0.3) (layer "F.Cu") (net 8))
 (via (at 179.66 113.29) (size 0.8) (drill 0.4) (layers "F.Cu" "B.Cu") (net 8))
 (via (at 167.81 118.39) (size 0.8) (drill 0.4) (layers "F.Cu" "B.Cu") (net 8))
 (segment (start 179.21 113.29) (end 179.66 113.29) (width 0.5) (layer "B.Cu") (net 8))
 (segment (start 167.81 118.39) (end 174.11 118.39) (width 0.5) (layer "B.Cu") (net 8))
 (segment (start 174.11 118.39) (end 179.21 113.29) (width 0.5) (layer "B.Cu") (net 8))
 (segment (start 174.88 113.71) (end 172.51 111.34) (width 0.3) (layer "F.Cu") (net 7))
 (segment (start 172.51 111.34) (end 172.0275 111.34) (width 0.3) (layer "F.Cu") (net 7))
 (segment (start 178.23 113.71) (end 174.88 113.71) (width 0.3) (layer "F.Cu") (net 7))
 (segment (start 178.23 115.21) (end 174.0725 115.21) (width 0.3) (layer "F.Cu") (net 4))
 (segment (start 174.0725 115.21) (end 172.0275 113.165) (width 0.3) (layer "F.Cu") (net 4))
 (segment (start 173.67307 115.71) (end 172.95307 114.99) (width 0.3) (layer "F.Cu") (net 3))
 (segment (start 178.23 115.71) (end 173.67307 115.71) (width 0.3) (layer "F.Cu") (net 3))
 (segment (start 172.95307 114.99) (end 172.0275 114.99) (width 0.3) (layer "F.Cu") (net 3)))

